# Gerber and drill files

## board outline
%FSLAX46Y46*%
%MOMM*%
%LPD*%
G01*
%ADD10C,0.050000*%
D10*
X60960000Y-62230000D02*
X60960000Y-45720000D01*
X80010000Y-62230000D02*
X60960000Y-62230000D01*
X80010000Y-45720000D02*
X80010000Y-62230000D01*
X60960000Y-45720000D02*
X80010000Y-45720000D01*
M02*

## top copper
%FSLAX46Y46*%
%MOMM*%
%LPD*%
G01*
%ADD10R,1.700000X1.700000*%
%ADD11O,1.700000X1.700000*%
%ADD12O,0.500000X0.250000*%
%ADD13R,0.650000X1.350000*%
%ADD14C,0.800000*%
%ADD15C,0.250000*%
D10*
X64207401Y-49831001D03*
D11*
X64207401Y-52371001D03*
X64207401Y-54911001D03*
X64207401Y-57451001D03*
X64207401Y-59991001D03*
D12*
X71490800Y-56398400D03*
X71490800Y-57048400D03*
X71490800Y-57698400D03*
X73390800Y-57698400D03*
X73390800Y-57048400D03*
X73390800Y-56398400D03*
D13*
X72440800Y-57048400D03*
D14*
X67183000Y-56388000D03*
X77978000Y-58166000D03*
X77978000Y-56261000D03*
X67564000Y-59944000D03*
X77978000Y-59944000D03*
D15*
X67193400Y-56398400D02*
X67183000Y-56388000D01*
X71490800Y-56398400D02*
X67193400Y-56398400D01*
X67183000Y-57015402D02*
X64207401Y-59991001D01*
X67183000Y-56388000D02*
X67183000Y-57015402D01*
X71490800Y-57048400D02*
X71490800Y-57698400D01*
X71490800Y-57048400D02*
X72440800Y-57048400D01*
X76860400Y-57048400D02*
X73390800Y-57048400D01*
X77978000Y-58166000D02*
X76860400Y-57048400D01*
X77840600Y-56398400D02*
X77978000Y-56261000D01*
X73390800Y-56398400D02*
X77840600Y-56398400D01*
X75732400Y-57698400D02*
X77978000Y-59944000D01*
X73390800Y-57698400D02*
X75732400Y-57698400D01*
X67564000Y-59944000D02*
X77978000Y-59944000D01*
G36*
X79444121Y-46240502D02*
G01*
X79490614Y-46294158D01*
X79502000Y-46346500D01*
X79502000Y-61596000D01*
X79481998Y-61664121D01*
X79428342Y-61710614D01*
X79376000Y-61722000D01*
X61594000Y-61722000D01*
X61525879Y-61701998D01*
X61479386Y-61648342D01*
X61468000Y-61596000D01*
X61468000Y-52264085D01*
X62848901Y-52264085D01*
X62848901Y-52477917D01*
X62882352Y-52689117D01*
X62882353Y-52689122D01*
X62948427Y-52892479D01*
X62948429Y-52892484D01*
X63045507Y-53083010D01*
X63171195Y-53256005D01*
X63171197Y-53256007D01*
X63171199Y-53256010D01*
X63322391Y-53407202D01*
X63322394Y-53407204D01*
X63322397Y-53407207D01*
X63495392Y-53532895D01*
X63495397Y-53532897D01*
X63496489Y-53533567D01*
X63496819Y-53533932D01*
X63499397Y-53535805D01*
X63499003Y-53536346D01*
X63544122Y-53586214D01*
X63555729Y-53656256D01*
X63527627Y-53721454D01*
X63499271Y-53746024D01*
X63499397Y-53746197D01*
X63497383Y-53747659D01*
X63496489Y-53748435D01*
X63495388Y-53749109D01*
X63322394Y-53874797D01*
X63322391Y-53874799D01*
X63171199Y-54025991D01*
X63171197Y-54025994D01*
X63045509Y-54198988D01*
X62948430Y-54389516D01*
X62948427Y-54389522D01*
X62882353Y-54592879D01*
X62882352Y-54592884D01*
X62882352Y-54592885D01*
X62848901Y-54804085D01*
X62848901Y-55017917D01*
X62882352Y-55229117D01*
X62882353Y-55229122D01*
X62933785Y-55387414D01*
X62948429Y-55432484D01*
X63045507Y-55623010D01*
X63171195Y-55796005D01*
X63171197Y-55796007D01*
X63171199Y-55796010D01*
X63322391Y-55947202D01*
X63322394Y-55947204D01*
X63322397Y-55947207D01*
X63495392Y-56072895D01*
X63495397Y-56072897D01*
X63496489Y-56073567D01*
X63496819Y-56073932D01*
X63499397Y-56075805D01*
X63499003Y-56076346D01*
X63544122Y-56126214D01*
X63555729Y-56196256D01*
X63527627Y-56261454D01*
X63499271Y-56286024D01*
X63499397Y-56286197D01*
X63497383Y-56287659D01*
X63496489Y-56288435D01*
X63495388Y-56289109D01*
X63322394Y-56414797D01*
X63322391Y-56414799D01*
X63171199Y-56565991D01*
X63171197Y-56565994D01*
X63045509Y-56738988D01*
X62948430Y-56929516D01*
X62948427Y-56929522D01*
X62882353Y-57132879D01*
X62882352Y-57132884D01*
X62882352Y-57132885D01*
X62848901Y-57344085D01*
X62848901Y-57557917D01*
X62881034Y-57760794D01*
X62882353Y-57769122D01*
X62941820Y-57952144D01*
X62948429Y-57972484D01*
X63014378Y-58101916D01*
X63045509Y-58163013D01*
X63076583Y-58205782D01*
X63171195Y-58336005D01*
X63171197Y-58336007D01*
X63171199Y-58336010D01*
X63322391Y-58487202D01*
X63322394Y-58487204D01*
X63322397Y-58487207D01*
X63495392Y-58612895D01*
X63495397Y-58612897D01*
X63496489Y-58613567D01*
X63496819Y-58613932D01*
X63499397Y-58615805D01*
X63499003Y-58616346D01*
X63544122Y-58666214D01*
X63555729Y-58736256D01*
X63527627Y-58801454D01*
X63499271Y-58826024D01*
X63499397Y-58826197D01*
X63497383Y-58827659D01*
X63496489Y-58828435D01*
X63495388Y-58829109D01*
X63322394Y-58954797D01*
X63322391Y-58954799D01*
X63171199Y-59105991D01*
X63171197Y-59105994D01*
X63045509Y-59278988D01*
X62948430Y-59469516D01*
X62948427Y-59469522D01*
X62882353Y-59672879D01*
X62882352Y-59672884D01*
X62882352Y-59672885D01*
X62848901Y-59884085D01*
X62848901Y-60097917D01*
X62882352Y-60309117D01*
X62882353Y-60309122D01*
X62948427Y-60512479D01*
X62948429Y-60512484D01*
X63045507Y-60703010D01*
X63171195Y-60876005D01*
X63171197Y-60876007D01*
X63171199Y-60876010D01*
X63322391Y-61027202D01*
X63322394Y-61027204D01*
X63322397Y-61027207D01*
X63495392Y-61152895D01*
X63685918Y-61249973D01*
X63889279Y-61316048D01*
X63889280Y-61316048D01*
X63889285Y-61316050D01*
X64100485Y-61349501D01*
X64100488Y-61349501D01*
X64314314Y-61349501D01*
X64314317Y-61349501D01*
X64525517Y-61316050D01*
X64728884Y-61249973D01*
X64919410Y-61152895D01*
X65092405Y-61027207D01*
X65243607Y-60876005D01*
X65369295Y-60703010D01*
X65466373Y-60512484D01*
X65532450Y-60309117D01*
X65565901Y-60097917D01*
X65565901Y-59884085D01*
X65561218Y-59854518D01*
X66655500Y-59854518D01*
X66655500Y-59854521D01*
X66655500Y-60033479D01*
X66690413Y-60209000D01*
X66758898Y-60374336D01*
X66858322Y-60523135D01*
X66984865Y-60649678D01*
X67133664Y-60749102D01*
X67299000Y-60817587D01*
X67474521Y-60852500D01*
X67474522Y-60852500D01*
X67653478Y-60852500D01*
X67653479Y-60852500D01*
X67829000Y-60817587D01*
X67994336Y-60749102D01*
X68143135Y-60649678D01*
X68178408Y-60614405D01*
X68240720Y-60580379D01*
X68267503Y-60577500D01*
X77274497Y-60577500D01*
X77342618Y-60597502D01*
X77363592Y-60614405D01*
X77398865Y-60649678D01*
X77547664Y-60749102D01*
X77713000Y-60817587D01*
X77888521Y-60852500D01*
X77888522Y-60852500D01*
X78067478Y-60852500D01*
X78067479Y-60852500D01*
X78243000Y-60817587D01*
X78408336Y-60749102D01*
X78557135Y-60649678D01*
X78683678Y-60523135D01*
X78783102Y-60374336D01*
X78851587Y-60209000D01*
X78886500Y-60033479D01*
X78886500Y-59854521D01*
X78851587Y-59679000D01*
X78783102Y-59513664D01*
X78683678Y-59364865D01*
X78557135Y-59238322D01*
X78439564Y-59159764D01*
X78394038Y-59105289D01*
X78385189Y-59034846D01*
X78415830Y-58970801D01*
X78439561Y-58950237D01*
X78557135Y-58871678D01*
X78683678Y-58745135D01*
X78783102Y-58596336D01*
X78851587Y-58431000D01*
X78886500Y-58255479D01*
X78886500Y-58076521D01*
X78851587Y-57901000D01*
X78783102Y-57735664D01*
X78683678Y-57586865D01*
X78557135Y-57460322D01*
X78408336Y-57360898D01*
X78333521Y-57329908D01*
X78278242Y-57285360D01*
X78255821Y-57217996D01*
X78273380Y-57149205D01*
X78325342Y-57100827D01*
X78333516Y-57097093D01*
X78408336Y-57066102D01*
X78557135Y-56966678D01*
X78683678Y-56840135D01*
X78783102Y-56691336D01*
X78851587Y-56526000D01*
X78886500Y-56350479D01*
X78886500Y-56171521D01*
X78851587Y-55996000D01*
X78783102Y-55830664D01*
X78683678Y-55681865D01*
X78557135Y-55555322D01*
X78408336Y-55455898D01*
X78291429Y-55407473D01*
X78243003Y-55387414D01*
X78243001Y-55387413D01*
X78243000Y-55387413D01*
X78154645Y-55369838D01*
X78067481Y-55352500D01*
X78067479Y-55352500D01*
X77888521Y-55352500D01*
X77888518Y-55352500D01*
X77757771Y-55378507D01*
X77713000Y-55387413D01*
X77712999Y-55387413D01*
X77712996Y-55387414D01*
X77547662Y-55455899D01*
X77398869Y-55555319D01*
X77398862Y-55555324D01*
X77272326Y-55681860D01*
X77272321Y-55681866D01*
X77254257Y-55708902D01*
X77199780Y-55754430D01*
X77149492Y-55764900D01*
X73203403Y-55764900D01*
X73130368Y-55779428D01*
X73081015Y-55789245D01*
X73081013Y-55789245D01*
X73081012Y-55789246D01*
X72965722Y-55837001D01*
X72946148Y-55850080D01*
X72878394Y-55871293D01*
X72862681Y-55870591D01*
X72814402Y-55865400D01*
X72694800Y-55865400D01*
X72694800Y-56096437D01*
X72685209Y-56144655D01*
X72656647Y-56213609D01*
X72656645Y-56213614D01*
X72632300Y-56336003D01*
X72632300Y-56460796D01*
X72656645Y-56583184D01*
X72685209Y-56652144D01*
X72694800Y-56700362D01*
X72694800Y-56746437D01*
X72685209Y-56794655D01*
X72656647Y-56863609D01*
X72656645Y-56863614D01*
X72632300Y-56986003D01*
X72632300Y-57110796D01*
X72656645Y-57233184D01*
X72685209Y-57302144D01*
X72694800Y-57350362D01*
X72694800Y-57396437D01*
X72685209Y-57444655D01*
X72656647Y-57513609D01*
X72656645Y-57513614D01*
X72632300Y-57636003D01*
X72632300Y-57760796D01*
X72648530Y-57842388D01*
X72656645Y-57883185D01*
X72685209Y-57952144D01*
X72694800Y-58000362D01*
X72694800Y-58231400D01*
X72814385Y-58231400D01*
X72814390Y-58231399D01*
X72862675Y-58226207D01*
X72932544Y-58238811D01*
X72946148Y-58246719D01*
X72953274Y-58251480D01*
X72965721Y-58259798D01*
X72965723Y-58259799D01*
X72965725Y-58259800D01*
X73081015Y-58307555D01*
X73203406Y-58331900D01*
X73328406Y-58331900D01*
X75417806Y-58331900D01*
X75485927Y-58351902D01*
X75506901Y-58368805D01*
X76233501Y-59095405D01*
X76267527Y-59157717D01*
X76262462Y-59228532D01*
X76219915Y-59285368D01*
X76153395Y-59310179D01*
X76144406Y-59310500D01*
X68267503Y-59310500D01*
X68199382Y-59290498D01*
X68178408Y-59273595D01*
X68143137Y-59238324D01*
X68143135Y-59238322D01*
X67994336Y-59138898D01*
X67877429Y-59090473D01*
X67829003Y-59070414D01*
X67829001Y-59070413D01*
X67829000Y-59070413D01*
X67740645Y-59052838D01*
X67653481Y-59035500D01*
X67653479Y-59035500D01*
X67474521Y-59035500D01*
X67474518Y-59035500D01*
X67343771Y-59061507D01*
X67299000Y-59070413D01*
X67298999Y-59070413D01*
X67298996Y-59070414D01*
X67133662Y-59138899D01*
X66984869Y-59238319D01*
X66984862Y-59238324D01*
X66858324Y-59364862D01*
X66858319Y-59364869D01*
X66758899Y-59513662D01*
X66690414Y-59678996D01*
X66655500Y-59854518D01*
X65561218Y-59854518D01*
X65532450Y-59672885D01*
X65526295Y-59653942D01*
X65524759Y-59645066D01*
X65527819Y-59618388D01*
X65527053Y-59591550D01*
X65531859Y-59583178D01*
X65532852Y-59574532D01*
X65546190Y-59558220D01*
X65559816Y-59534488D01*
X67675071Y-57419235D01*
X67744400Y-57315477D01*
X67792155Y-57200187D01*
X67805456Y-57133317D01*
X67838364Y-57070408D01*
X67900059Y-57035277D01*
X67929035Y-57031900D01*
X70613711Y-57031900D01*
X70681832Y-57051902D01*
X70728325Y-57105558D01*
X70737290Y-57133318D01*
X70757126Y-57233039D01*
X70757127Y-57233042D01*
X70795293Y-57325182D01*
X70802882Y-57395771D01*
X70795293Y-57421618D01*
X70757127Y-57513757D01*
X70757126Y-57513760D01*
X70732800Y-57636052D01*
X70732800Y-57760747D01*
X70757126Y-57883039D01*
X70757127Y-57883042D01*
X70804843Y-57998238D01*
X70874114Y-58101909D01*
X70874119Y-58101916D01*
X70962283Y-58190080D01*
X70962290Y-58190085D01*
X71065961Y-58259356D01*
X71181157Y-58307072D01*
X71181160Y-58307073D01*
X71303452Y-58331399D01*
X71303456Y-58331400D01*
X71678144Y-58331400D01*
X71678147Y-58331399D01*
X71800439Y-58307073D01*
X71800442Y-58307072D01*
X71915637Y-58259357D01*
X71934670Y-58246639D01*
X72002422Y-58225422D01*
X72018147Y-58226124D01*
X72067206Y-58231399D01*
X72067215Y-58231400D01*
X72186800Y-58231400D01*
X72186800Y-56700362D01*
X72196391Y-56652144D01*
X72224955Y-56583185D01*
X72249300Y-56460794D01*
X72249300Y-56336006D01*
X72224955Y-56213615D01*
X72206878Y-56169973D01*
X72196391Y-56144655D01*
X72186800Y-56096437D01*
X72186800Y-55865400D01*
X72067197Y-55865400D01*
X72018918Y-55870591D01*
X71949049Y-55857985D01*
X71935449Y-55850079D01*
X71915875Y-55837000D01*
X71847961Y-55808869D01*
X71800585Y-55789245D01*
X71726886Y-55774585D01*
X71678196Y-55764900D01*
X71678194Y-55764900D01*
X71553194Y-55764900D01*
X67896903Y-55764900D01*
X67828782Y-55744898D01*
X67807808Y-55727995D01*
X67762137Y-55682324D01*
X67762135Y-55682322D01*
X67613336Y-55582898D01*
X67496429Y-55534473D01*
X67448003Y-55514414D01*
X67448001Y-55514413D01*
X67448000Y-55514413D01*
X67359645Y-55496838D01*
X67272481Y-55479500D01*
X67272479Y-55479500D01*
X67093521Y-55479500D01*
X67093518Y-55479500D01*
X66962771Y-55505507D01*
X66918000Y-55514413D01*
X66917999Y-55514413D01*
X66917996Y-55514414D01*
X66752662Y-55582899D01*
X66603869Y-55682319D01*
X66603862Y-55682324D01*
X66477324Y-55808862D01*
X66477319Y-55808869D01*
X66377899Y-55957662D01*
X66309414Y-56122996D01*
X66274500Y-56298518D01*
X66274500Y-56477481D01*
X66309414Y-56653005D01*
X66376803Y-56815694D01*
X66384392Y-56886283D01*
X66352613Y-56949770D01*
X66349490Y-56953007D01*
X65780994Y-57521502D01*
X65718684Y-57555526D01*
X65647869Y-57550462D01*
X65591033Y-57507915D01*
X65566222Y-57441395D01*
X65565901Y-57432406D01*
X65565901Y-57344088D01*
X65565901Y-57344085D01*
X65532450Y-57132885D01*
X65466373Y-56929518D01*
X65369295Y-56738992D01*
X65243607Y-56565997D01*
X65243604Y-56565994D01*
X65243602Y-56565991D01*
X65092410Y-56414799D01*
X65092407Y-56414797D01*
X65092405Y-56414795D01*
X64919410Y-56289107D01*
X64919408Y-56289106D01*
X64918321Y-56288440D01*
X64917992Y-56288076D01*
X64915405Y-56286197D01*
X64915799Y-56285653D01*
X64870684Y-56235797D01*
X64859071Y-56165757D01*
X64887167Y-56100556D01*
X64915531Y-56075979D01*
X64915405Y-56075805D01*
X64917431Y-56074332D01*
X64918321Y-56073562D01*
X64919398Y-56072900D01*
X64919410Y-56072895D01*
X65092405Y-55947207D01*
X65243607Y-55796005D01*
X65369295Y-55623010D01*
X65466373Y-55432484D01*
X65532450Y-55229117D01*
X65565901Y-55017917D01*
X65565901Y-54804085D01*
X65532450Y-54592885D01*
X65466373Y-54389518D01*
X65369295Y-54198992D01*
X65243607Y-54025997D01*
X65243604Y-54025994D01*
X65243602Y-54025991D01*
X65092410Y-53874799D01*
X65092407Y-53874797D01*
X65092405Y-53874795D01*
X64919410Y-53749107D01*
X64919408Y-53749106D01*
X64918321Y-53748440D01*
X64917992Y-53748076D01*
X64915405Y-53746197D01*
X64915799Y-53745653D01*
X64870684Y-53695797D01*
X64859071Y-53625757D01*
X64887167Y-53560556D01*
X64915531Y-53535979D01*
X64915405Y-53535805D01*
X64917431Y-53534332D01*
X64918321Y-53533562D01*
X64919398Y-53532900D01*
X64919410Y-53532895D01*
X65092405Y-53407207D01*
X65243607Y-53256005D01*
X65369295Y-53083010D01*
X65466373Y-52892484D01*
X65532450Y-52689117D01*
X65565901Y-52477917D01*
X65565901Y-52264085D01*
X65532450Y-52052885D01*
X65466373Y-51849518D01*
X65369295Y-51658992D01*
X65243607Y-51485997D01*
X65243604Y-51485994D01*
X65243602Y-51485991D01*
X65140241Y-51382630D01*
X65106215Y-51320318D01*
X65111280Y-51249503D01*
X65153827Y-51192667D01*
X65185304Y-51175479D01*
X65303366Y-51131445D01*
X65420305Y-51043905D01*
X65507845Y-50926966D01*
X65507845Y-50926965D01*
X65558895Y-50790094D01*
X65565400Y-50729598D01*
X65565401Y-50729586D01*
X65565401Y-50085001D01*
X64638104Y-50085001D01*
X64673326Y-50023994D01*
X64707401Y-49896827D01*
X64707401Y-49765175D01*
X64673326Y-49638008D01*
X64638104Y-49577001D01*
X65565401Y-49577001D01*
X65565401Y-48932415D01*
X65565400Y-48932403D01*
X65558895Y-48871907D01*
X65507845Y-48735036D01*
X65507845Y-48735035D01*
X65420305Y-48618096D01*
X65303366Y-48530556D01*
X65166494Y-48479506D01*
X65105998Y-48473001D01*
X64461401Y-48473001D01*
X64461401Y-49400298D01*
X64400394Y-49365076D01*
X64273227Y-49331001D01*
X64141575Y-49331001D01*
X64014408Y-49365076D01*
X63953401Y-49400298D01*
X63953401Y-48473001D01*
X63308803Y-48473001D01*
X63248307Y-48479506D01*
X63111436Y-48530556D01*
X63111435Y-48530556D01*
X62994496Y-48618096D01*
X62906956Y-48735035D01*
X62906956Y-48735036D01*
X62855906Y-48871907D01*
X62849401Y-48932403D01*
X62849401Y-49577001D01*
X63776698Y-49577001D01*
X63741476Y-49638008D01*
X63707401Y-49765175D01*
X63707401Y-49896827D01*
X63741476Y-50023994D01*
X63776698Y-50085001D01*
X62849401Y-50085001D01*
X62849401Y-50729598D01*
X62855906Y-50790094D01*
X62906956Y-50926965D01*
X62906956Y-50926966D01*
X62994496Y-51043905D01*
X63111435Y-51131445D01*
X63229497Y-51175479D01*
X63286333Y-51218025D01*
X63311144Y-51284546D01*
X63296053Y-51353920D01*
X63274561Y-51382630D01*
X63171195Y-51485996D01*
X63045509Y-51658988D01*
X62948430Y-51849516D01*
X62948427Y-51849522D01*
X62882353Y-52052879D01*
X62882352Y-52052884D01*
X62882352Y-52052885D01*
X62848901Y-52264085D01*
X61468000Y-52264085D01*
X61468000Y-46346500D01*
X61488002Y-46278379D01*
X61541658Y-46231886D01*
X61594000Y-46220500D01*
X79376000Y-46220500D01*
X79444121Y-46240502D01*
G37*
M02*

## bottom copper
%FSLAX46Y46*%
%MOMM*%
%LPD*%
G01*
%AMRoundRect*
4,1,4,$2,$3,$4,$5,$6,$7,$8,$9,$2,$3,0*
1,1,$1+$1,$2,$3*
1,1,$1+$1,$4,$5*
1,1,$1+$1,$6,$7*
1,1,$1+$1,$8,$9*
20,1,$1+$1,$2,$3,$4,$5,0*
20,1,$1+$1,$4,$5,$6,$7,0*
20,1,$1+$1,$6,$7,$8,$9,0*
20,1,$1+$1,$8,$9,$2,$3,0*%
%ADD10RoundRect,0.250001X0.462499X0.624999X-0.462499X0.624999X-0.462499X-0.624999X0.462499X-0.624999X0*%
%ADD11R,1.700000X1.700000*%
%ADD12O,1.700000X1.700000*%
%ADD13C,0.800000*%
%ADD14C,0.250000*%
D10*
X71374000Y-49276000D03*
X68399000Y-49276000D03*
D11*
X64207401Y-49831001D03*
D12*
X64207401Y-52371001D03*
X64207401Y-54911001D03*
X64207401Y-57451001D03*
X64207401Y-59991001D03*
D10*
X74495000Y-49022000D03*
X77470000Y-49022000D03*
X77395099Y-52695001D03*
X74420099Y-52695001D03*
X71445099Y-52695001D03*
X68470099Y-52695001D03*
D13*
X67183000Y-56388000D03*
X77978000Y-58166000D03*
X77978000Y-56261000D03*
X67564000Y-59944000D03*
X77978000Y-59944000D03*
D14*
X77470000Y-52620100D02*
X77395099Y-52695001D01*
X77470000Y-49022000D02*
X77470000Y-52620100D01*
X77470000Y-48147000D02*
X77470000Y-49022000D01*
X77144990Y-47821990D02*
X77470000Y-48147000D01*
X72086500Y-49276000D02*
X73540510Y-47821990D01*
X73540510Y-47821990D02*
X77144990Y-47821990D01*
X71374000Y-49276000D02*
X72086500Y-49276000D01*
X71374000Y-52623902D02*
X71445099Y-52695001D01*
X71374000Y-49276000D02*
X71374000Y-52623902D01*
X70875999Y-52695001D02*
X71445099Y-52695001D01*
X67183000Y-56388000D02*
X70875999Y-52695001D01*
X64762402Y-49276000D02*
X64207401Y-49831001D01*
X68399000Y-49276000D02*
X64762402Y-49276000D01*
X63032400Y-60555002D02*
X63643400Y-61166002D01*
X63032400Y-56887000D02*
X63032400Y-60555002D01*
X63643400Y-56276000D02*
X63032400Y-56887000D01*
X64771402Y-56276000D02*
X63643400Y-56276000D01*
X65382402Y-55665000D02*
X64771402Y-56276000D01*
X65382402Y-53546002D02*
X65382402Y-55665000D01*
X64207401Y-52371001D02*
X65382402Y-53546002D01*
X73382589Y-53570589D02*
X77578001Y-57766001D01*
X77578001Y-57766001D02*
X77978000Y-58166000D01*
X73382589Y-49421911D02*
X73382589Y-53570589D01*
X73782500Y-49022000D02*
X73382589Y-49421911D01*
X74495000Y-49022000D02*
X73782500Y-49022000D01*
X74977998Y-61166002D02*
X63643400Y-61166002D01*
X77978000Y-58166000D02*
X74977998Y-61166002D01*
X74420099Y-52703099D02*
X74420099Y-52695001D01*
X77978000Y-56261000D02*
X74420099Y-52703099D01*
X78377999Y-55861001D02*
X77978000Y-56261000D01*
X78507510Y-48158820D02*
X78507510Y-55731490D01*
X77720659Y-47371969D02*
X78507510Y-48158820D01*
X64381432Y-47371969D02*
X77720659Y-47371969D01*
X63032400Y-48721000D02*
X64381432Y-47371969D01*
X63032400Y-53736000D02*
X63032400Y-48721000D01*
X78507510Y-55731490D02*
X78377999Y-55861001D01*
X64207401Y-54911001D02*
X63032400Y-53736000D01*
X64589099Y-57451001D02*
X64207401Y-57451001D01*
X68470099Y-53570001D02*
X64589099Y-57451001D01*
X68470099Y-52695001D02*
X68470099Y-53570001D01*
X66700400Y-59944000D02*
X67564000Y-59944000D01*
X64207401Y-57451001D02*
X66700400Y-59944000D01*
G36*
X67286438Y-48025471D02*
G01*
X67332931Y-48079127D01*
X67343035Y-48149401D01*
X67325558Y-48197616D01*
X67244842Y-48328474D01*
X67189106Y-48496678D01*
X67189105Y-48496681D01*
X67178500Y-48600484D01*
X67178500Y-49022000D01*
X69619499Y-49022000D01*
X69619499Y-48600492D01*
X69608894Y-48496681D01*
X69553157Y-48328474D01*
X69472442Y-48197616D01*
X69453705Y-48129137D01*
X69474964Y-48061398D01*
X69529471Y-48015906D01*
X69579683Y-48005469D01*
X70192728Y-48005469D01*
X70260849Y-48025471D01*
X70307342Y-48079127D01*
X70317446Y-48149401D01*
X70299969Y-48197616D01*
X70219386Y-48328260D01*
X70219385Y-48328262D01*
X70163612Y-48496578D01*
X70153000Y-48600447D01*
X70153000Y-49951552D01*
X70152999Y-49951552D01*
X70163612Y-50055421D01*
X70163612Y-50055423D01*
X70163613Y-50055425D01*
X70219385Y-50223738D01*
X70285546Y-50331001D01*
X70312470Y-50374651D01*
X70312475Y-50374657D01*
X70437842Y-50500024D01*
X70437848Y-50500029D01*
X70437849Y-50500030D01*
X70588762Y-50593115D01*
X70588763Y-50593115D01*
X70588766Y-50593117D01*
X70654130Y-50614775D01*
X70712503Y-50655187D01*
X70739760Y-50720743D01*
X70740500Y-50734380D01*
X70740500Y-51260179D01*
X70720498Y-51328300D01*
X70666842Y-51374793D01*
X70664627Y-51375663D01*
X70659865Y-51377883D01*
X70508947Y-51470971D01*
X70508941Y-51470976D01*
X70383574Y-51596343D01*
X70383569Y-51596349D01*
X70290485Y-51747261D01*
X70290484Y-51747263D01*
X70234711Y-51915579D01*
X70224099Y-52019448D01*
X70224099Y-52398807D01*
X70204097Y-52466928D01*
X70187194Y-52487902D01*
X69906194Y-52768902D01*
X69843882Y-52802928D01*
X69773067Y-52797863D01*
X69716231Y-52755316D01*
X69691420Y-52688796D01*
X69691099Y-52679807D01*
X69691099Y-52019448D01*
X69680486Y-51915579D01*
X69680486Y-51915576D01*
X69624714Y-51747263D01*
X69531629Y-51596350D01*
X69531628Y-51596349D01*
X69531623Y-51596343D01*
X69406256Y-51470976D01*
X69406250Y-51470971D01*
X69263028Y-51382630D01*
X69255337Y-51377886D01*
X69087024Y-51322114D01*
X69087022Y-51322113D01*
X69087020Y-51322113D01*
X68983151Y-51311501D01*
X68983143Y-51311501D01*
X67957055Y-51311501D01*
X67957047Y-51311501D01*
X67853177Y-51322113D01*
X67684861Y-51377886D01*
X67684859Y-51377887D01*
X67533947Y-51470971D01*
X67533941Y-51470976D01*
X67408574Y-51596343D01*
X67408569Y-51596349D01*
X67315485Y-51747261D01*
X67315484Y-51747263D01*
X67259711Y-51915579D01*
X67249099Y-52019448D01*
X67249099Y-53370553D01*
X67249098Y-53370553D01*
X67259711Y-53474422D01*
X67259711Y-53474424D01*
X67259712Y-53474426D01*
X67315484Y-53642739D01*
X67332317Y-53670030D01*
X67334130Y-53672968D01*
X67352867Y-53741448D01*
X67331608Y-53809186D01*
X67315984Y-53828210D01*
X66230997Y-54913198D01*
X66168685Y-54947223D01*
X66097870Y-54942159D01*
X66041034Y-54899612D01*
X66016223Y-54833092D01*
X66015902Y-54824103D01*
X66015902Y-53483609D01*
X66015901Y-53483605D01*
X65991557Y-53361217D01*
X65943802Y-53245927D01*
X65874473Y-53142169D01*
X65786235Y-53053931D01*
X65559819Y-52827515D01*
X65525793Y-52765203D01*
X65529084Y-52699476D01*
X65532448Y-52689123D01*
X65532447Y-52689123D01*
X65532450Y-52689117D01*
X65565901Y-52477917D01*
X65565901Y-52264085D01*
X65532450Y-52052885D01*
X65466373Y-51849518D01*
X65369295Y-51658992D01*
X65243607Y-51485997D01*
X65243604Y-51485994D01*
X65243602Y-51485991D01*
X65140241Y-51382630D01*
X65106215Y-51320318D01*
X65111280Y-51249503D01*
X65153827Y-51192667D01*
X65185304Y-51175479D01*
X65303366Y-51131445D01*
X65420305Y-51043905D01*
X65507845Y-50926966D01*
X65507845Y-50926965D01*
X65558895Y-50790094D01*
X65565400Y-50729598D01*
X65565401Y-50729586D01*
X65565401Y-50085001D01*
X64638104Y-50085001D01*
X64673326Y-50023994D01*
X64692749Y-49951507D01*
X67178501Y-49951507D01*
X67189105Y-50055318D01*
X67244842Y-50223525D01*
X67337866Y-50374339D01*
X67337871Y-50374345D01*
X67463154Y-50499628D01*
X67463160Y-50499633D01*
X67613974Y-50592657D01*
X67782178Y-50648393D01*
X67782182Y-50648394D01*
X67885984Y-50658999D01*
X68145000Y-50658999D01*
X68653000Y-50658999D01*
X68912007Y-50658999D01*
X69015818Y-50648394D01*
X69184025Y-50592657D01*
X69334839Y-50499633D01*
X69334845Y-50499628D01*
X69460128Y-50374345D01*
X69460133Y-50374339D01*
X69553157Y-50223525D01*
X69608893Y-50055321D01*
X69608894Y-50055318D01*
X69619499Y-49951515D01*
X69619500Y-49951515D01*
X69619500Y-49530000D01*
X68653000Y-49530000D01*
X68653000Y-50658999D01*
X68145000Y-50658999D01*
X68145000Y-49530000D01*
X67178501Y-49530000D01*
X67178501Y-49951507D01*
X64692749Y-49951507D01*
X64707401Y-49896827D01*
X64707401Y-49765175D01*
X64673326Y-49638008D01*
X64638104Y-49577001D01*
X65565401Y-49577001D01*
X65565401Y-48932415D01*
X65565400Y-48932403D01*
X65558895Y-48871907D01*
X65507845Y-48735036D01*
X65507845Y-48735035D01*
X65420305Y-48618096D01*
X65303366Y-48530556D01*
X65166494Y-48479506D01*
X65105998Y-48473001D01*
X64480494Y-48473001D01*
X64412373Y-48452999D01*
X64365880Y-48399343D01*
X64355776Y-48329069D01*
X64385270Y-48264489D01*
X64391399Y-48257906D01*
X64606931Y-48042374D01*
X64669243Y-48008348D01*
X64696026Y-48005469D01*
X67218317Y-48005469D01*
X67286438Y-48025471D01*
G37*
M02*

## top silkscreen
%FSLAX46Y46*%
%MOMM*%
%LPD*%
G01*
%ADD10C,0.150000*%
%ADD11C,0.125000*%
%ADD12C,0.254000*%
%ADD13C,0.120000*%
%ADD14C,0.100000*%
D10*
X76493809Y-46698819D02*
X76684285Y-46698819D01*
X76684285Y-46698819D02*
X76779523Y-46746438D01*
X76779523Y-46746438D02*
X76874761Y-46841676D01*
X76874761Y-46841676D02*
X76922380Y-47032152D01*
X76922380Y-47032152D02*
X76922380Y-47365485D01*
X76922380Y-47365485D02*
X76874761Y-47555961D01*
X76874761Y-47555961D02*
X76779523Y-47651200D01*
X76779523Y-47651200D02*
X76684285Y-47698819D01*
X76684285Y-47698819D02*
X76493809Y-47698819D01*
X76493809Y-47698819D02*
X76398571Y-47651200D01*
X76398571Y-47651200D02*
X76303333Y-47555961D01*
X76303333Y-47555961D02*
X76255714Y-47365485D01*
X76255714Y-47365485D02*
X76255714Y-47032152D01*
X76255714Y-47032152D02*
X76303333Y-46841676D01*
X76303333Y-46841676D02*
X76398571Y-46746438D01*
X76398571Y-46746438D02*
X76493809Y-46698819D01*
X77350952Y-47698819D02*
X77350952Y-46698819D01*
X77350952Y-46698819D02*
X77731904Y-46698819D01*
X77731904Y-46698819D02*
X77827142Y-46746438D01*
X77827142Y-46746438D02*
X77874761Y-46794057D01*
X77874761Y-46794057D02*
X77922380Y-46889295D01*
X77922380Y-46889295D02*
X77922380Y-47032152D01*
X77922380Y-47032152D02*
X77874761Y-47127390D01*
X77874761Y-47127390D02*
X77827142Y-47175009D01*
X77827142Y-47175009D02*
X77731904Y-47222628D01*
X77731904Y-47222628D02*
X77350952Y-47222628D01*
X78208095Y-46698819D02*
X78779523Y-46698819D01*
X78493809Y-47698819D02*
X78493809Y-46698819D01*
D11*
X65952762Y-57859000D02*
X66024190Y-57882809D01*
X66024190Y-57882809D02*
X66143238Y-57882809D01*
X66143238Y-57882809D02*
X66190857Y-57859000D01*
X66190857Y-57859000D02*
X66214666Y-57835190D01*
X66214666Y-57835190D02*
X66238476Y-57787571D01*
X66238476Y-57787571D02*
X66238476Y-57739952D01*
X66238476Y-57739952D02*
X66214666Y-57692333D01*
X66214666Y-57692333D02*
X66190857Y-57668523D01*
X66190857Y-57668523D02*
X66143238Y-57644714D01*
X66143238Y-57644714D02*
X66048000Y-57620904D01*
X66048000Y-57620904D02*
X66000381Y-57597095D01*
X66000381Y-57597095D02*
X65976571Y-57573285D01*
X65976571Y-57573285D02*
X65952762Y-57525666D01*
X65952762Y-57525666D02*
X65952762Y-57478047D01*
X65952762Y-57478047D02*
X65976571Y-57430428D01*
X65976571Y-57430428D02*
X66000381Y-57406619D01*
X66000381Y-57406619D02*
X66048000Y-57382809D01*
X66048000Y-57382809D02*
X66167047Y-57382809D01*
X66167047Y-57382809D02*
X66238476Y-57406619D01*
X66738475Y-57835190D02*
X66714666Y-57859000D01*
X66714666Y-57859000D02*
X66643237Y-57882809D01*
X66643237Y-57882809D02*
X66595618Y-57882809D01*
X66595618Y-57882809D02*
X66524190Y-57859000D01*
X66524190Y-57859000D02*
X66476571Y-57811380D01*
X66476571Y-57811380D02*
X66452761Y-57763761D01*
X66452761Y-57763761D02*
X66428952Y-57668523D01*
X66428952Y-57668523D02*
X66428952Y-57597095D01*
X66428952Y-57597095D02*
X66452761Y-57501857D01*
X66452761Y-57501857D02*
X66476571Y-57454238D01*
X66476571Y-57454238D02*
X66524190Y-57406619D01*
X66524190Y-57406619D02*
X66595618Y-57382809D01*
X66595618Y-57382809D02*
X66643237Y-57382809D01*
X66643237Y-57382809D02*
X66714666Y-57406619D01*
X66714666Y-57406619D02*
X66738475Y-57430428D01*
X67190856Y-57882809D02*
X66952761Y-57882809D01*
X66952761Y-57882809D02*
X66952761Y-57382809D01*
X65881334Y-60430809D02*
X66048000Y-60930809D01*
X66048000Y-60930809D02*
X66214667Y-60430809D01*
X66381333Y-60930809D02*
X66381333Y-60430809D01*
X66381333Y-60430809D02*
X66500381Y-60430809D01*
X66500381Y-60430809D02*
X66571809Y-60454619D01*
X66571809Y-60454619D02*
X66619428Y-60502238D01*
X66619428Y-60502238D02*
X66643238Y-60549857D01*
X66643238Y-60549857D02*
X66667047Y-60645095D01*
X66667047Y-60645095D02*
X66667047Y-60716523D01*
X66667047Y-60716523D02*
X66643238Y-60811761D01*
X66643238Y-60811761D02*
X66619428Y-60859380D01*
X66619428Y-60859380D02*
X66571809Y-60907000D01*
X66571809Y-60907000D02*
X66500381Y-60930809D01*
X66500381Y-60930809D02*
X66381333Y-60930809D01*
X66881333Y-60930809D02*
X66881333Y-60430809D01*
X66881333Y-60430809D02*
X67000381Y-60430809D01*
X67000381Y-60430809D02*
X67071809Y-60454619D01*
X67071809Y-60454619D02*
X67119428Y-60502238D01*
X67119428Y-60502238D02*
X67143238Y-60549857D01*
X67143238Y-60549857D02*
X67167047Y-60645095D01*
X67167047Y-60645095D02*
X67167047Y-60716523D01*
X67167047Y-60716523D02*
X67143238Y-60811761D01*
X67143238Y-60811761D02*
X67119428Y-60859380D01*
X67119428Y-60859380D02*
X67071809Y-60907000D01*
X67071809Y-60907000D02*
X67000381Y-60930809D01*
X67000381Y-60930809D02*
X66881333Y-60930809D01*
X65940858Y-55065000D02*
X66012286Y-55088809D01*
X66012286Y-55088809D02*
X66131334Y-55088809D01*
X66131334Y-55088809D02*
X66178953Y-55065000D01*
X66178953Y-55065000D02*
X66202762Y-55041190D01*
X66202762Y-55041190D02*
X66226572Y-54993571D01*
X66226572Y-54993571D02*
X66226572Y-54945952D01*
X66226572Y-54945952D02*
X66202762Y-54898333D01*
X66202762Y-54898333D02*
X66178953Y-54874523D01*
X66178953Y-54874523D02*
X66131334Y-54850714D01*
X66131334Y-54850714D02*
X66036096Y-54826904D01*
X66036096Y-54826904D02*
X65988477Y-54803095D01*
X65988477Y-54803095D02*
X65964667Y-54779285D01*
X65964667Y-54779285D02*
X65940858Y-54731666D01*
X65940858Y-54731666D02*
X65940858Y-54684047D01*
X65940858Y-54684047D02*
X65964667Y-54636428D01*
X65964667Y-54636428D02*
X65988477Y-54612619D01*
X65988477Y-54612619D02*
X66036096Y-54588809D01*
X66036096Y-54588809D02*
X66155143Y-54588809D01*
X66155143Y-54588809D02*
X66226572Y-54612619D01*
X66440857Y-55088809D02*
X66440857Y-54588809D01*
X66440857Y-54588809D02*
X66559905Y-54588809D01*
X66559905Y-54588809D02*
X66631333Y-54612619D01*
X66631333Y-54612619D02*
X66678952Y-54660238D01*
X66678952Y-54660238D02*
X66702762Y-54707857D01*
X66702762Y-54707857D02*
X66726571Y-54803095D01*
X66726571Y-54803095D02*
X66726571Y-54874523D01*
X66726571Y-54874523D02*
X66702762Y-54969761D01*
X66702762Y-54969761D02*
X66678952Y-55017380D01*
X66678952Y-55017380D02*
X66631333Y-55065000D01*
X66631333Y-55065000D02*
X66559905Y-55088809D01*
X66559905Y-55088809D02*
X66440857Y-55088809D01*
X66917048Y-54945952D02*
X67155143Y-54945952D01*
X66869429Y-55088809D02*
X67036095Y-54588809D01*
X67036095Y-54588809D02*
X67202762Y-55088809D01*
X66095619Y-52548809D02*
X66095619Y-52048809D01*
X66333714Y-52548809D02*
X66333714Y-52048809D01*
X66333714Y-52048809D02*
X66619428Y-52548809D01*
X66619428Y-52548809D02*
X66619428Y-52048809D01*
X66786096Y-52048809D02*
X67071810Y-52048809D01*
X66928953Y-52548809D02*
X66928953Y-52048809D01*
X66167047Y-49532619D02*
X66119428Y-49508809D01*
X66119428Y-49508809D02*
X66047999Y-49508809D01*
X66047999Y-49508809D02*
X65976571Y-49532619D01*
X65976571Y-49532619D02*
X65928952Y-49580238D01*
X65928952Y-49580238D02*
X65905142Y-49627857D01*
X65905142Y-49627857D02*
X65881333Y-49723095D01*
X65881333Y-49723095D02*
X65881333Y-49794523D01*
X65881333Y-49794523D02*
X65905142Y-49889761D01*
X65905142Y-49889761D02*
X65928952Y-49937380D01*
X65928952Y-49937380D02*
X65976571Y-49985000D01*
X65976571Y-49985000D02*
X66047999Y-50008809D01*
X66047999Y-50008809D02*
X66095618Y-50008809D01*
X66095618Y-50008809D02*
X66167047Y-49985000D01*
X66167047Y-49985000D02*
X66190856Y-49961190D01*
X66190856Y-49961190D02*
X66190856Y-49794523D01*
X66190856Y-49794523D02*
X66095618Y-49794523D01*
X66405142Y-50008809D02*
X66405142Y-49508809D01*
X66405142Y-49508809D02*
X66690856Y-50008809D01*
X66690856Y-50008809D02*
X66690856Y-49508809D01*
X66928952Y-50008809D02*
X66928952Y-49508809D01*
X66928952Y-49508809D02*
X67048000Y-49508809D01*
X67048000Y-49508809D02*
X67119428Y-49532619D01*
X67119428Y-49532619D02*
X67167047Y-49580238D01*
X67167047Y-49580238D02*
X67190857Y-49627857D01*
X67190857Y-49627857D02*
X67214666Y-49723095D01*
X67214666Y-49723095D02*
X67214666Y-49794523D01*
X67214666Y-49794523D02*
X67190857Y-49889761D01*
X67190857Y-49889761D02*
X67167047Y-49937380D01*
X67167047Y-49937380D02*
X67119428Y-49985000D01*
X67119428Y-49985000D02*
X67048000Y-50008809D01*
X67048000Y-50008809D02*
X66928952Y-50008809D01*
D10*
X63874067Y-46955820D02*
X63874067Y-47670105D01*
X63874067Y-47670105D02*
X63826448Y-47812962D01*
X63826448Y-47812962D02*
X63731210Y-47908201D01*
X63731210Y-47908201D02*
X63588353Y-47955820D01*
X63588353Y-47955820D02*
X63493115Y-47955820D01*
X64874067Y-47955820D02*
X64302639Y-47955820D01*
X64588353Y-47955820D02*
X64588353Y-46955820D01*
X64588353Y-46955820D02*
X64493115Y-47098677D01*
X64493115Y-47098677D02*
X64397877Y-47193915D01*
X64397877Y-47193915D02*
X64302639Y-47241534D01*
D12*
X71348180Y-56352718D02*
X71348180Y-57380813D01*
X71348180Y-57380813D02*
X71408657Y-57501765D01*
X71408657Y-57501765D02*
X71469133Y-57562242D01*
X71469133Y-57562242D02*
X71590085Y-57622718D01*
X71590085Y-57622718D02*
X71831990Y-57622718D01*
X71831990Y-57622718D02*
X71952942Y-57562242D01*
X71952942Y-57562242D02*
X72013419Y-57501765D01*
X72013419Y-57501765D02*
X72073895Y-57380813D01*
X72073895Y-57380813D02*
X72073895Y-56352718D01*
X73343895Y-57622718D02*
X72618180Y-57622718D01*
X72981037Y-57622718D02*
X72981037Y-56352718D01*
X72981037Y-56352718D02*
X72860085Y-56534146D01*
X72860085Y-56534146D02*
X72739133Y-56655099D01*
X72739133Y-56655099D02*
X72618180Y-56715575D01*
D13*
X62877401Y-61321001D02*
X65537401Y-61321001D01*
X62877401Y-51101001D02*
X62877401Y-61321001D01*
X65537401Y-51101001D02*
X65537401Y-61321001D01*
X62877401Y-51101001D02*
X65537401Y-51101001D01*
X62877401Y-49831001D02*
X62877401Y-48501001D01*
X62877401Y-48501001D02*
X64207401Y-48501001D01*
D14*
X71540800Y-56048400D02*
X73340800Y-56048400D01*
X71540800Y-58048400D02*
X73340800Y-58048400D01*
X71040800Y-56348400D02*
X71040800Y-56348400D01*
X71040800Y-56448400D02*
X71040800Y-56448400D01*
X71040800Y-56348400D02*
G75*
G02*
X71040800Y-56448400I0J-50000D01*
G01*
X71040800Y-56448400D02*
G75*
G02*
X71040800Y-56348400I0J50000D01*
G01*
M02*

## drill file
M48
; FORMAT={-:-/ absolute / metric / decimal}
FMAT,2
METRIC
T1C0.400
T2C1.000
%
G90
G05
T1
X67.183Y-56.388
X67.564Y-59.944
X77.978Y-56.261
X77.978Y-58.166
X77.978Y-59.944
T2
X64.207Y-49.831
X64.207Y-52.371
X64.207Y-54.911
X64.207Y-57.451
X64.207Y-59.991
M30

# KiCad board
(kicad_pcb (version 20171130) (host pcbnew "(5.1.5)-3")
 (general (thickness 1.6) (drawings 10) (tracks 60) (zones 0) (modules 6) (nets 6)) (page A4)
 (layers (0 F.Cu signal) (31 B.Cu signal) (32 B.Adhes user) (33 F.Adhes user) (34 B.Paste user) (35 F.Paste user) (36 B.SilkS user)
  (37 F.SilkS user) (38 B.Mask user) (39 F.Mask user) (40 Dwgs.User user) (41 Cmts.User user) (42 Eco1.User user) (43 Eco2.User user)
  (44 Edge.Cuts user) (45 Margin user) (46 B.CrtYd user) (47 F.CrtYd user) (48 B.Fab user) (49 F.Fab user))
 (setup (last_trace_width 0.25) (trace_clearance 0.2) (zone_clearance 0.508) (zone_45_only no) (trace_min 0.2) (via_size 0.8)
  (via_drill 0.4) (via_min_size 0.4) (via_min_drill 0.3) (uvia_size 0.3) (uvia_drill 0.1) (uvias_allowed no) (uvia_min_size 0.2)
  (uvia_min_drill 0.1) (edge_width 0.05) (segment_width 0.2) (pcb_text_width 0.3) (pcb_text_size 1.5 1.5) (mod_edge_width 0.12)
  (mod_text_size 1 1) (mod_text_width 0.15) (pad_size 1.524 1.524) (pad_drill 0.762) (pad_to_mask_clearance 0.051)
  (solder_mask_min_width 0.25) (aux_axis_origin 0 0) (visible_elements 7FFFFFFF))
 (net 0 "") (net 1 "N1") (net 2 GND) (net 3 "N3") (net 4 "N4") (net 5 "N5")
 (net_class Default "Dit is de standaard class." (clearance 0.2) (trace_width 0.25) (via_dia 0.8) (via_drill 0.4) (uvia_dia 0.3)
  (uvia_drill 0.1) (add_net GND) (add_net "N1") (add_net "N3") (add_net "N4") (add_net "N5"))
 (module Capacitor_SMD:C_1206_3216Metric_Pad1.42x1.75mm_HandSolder (layer B.Cu) (at 69.8865 49.276 180)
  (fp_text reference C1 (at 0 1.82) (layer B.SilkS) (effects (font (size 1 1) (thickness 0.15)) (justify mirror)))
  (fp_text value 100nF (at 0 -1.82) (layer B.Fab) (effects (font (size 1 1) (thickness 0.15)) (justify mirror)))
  (pad 1 smd roundrect (at -1.4875 0 180) (size 1.425 1.75) (layers B.Cu B.Paste B.Mask) (roundrect_rratio 0.175439) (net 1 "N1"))
  (pad 2 smd roundrect (at 1.4875 0 180) (size 1.425 1.75) (layers B.Cu B.Paste B.Mask) (roundrect_rratio 0.175439) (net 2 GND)))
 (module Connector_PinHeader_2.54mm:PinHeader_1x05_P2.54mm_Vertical (layer F.Cu) (at 64.207401 49.831001)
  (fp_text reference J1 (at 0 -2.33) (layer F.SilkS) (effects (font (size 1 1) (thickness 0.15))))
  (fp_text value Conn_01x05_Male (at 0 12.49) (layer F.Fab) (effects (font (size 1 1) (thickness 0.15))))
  (fp_line (start -1.33 11.49) (end 1.33 11.49) (layer F.SilkS) (width 0.12))
  (fp_line (start -1.33 1.27) (end -1.33 11.49) (layer F.SilkS) (width 0.12))
  (fp_line (start 1.33 1.27) (end 1.33 11.49) (layer F.SilkS) (width 0.12))
  (fp_line (start -1.33 1.27) (end 1.33 1.27) (layer F.SilkS) (width 0.12))
  (fp_line (start -1.33 0) (end -1.33 -1.33) (layer F.SilkS) (width 0.12))
  (fp_line (start -1.33 -1.33) (end 0 -1.33) (layer F.SilkS) (width 0.12))
  (pad 1 thru_hole rect (at 0 0) (size 1.7 1.7) (drill 1) (layers *.Cu *.Mask) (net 2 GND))
  (pad 2 thru_hole oval (at 0 2.54) (size 1.7 1.7) (drill 1) (layers *.Cu *.Mask) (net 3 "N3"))
  (pad 3 thru_hole oval (at 0 5.08) (size 1.7 1.7) (drill 1) (layers *.Cu *.Mask) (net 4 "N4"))
  (pad 4 thru_hole oval (at 0 7.62) (size 1.7 1.7) (drill 1) (layers *.Cu *.Mask) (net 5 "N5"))
  (pad 5 thru_hole oval (at 0 10.16) (size 1.7 1.7) (drill 1) (layers *.Cu *.Mask) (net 1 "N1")))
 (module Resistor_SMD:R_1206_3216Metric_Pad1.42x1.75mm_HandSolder (layer B.Cu) (at 75.9825 49.022 180)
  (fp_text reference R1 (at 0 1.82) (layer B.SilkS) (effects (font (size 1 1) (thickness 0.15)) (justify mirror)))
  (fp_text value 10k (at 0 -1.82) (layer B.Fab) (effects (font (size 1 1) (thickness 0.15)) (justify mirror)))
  (pad 2 smd roundrect (at 1.4875 0 180) (size 1.425 1.75) (layers B.Cu B.Paste B.Mask) (roundrect_rratio 0.175439) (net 3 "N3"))
  (pad 1 smd roundrect (at -1.4875 0 180) (size 1.425 1.75) (layers B.Cu B.Paste B.Mask) (roundrect_rratio 0.175439) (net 1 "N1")))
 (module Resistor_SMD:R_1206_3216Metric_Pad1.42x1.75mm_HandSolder (layer B.Cu) (at 75.907599 52.695001 180)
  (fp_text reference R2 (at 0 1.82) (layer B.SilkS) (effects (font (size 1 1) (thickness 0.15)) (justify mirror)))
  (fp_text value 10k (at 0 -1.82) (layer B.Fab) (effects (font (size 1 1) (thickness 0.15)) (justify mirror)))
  (pad 1 smd roundrect (at -1.4875 0 180) (size 1.425 1.75) (layers B.Cu B.Paste B.Mask) (roundrect_rratio 0.175439) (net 1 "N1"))
  (pad 2 smd roundrect (at 1.4875 0 180) (size 1.425 1.75) (layers B.Cu B.Paste B.Mask) (roundrect_rratio 0.175439) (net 4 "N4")))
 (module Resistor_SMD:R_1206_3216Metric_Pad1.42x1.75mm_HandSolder (layer B.Cu) (at 69.957599 52.695001 180)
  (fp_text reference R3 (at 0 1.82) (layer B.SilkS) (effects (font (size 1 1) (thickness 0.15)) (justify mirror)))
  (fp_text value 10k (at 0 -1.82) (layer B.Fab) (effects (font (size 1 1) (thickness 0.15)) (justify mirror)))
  (pad 1 smd roundrect (at -1.4875 0 180) (size 1.425 1.75) (layers B.Cu B.Paste B.Mask) (roundrect_rratio 0.175439) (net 1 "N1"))
  (pad 2 smd roundrect (at 1.4875 0 180) (size 1.425 1.75) (layers B.Cu B.Paste B.Mask) (roundrect_rratio 0.175439) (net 5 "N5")))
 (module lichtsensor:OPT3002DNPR (layer F.Cu) (at 72.3158 57.0484)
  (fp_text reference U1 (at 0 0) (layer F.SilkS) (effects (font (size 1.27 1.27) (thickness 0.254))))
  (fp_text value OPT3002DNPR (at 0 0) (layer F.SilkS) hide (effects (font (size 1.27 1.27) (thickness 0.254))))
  (fp_line (start -0.775 -1) (end 1.025 -1) (layer F.SilkS) (width 0.1))
  (fp_line (start -0.775 1) (end 1.025 1) (layer F.SilkS) (width 0.1))
  (fp_line (start -1.275 -0.7) (end -1.275 -0.7) (layer F.SilkS) (width 0.1))
  (fp_line (start -1.275 -0.6) (end -1.275 -0.6) (layer F.SilkS) (width 0.1))
  (fp_arc (start -1.275 -0.65) (end -1.275 -0.7) (angle 180) (layer F.SilkS) (width 0.1))
  (fp_arc (start -1.275 -0.65) (end -1.275 -0.6) (angle 180) (layer F.SilkS) (width 0.1))
  (pad 1 smd oval (at -0.825 -0.65 90) (size 0.25 0.5) (layers F.Cu F.Paste F.Mask) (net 1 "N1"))
  (pad 2 smd oval (at -0.825 0 90) (size 0.25 0.5) (layers F.Cu F.Paste F.Mask) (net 2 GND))
  (pad 3 smd oval (at -0.825 0.65 90) (size 0.25 0.5) (layers F.Cu F.Paste F.Mask) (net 2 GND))
  (pad 4 smd oval (at 1.075 0.65 90) (size 0.25 0.5) (layers F.Cu F.Paste F.Mask) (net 5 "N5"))
  (pad 5 smd oval (at 1.075 0 90) (size 0.25 0.5) (layers F.Cu F.Paste F.Mask) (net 3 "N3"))
  (pad 6 smd oval (at 1.075 -0.65 90) (size 0.25 0.5) (layers F.Cu F.Paste F.Mask) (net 4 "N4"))
  (pad 7 smd rect (at 0.125 0) (size 0.65 1.35) (layers F.Cu F.Paste F.Mask) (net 2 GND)))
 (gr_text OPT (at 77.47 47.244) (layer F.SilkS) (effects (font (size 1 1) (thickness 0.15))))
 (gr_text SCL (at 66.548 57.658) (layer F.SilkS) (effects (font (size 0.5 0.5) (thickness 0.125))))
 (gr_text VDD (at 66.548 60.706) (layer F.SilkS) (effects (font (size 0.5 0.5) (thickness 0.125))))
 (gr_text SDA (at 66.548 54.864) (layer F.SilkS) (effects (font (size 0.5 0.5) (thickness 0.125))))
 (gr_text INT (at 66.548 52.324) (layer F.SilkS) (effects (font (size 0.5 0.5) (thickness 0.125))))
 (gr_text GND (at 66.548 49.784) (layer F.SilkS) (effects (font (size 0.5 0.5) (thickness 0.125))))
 (gr_line (start 60.96 62.23) (end 60.96 45.72) (layer Edge.Cuts) (width 0.05))
 (gr_line (start 80.01 62.23) (end 60.96 62.23) (layer Edge.Cuts) (width 0.05))
 (gr_line (start 80.01 45.72) (end 80.01 62.23) (layer Edge.Cuts) (width 0.05))
 (gr_line (start 60.96 45.72) (end 80.01 45.72) (layer Edge.Cuts) (width 0.05))
 (via (at 67.183 56.388) (size 0.8) (drill 0.4) (layers F.Cu B.Cu) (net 1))
 (segment (start 77.47 52.6201) (end 77.395099 52.695001) (width 0.25) (layer B.Cu) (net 1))
 (segment (start 77.47 49.022) (end 77.47 52.6201) (width 0.25) (layer B.Cu) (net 1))
 (segment (start 77.47 48.147) (end 77.47 49.022) (width 0.25) (layer B.Cu) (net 1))
 (segment (start 77.14499 47.82199) (end 77.47 48.147) (width 0.25) (layer B.Cu) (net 1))
 (segment (start 72.0865 49.276) (end 73.54051 47.82199) (width 0.25) (layer B.Cu) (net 1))
 (segment (start 73.54051 47.82199) (end 77.14499 47.82199) (width 0.25) (layer B.Cu) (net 1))
 (segment (start 71.374 49.276) (end 72.0865 49.276) (width 0.25) (layer B.Cu) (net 1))
 (segment (start 71.374 52.623902) (end 71.445099 52.695001) (width 0.25) (layer B.Cu) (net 1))
 (segment (start 71.374 49.276) (end 71.374 52.623902) (width 0.25) (layer B.Cu) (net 1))
 (segment (start 67.1934 56.3984) (end 67.183 56.388) (width 0.25) (layer F.Cu) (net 1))
 (segment (start 71.4908 56.3984) (end 67.1934 56.3984) (width 0.25) (layer F.Cu) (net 1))
 (segment (start 67.183 57.015402) (end 64.207401 59.991001) (width 0.25) (layer F.Cu) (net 1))
 (segment (start 67.183 56.388) (end 67.183 57.015402) (width 0.25) (layer F.Cu) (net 1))
 (segment (start 70.875999 52.695001) (end 71.445099 52.695001) (width 0.25) (layer B.Cu) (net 1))
 (segment (start 67.183 56.388) (end 70.875999 52.695001) (width 0.25) (layer B.Cu) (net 1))
 (segment (start 64.762402 49.276) (end 64.207401 49.831001) (width 0.25) (layer B.Cu) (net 2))
 (segment (start 68.399 49.276) (end 64.762402 49.276) (width 0.25) (layer B.Cu) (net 2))
 (segment (start 71.4908 57.0484) (end 71.4908 57.6984) (width 0.25) (layer F.Cu) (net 2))
 (segment (start 71.4908 57.0484) (end 72.4408 57.0484) (width 0.25) (layer F.Cu) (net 2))
 (via (at 77.978 58.166) (size 0.8) (drill 0.4) (layers F.Cu B.Cu) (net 3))
 (segment (start 63.0324 60.555002) (end 63.6434 61.166002) (width 0.25) (layer B.Cu) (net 3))
 (segment (start 63.0324 56.887) (end 63.0324 60.555002) (width 0.25) (layer B.Cu) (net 3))
 (segment (start 63.6434 56.276) (end 63.0324 56.887) (width 0.25) (layer B.Cu) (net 3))
 (segment (start 64.771402 56.276) (end 63.6434 56.276) (width 0.25) (layer B.Cu) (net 3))
 (segment (start 65.382402 55.665) (end 64.771402 56.276) (width 0.25) (layer B.Cu) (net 3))
 (segment (start 65.382402 53.546002) (end 65.382402 55.665) (width 0.25) (layer B.Cu) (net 3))
 (segment (start 64.207401 52.371001) (end 65.382402 53.546002) (width 0.25) (layer B.Cu) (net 3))
 (segment (start 76.8604 57.0484) (end 73.3908 57.0484) (width 0.25) (layer F.Cu) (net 3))
 (segment (start 77.978 58.166) (end 76.8604 57.0484) (width 0.25) (layer F.Cu) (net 3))
 (segment (start 73.382589 53.570589) (end 77.578001 57.766001) (width 0.25) (layer B.Cu) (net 3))
 (segment (start 77.578001 57.766001) (end 77.978 58.166) (width 0.25) (layer B.Cu) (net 3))
 (segment (start 73.382589 49.421911) (end 73.382589 53.570589) (width 0.25) (layer B.Cu) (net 3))
 (segment (start 73.7825 49.022) (end 73.382589 49.421911) (width 0.25) (layer B.Cu) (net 3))
 (segment (start 74.495 49.022) (end 73.7825 49.022) (width 0.25) (layer B.Cu) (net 3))
 (segment (start 74.977998 61.166002) (end 63.6434 61.166002) (width 0.25) (layer B.Cu) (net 3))
 (segment (start 77.978 58.166) (end 74.977998 61.166002) (width 0.25) (layer B.Cu) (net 3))
 (via (at 77.978 56.261) (size 0.8) (drill 0.4) (layers F.Cu B.Cu) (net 4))
 (segment (start 77.8406 56.3984) (end 77.978 56.261) (width 0.25) (layer F.Cu) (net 4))
 (segment (start 73.3908 56.3984) (end 77.8406 56.3984) (width 0.25) (layer F.Cu) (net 4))
 (segment (start 74.420099 52.703099) (end 74.420099 52.695001) (width 0.25) (layer B.Cu) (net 4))
 (segment (start 77.978 56.261) (end 74.420099 52.703099) (width 0.25) (layer B.Cu) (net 4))
 (segment (start 78.377999 55.861001) (end 77.978 56.261) (width 0.25) (layer B.Cu) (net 4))
 (segment (start 78.50751 48.15882) (end 78.50751 55.73149) (width 0.25) (layer B.Cu) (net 4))
 (segment (start 77.720659 47.371969) (end 78.50751 48.15882) (width 0.25) (layer B.Cu) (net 4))
 (segment (start 64.381432 47.371969) (end 77.720659 47.371969) (width 0.25) (layer B.Cu) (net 4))
 (segment (start 63.0324 48.721) (end 64.381432 47.371969) (width 0.25) (layer B.Cu) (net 4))
 (segment (start 63.0324 53.736) (end 63.0324 48.721) (width 0.25) (layer B.Cu) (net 4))
 (segment (start 78.50751 55.73149) (end 78.377999 55.861001) (width 0.25) (layer B.Cu) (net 4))
 (segment (start 64.207401 54.911001) (end 63.0324 53.736) (width 0.25) (layer B.Cu) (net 4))
 (via (at 67.564 59.944) (size 0.8) (drill 0.4) (layers F.Cu B.Cu) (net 5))
 (via (at 77.978 59.944) (size 0.8) (drill 0.4) (layers F.Cu B.Cu) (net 5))
 (segment (start 64.589099 57.451001) (end 64.207401 57.451001) (width 0.25) (layer B.Cu) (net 5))
 (segment (start 68.470099 53.570001) (end 64.589099 57.451001) (width 0.25) (layer B.Cu) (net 5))
 (segment (start 68.470099 52.695001) (end 68.470099 53.570001) (width 0.25) (layer B.Cu) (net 5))
 (segment (start 75.7324 57.6984) (end 77.978 59.944) (width 0.25) (layer F.Cu) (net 5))
 (segment (start 73.3908 57.6984) (end 75.7324 57.6984) (width 0.25) (layer F.Cu) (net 5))
 (segment (start 66.7004 59.944) (end 67.564 59.944) (width 0.25) (layer B.Cu) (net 5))
 (segment (start 64.207401 57.451001) (end 66.7004 59.944) (width 0.25) (layer B.Cu) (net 5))
 (segment (start 67.564 59.944) (end 77.978 59.944) (width 0.25) (layer F.Cu) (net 5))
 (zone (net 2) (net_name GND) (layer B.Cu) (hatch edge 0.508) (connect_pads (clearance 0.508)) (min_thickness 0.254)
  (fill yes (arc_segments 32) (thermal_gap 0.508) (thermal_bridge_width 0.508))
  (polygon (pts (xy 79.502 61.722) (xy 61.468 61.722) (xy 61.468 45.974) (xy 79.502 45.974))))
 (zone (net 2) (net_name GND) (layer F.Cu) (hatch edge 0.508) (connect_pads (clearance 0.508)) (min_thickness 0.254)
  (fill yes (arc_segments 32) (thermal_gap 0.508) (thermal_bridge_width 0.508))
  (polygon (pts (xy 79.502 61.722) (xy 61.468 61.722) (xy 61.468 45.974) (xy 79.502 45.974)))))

